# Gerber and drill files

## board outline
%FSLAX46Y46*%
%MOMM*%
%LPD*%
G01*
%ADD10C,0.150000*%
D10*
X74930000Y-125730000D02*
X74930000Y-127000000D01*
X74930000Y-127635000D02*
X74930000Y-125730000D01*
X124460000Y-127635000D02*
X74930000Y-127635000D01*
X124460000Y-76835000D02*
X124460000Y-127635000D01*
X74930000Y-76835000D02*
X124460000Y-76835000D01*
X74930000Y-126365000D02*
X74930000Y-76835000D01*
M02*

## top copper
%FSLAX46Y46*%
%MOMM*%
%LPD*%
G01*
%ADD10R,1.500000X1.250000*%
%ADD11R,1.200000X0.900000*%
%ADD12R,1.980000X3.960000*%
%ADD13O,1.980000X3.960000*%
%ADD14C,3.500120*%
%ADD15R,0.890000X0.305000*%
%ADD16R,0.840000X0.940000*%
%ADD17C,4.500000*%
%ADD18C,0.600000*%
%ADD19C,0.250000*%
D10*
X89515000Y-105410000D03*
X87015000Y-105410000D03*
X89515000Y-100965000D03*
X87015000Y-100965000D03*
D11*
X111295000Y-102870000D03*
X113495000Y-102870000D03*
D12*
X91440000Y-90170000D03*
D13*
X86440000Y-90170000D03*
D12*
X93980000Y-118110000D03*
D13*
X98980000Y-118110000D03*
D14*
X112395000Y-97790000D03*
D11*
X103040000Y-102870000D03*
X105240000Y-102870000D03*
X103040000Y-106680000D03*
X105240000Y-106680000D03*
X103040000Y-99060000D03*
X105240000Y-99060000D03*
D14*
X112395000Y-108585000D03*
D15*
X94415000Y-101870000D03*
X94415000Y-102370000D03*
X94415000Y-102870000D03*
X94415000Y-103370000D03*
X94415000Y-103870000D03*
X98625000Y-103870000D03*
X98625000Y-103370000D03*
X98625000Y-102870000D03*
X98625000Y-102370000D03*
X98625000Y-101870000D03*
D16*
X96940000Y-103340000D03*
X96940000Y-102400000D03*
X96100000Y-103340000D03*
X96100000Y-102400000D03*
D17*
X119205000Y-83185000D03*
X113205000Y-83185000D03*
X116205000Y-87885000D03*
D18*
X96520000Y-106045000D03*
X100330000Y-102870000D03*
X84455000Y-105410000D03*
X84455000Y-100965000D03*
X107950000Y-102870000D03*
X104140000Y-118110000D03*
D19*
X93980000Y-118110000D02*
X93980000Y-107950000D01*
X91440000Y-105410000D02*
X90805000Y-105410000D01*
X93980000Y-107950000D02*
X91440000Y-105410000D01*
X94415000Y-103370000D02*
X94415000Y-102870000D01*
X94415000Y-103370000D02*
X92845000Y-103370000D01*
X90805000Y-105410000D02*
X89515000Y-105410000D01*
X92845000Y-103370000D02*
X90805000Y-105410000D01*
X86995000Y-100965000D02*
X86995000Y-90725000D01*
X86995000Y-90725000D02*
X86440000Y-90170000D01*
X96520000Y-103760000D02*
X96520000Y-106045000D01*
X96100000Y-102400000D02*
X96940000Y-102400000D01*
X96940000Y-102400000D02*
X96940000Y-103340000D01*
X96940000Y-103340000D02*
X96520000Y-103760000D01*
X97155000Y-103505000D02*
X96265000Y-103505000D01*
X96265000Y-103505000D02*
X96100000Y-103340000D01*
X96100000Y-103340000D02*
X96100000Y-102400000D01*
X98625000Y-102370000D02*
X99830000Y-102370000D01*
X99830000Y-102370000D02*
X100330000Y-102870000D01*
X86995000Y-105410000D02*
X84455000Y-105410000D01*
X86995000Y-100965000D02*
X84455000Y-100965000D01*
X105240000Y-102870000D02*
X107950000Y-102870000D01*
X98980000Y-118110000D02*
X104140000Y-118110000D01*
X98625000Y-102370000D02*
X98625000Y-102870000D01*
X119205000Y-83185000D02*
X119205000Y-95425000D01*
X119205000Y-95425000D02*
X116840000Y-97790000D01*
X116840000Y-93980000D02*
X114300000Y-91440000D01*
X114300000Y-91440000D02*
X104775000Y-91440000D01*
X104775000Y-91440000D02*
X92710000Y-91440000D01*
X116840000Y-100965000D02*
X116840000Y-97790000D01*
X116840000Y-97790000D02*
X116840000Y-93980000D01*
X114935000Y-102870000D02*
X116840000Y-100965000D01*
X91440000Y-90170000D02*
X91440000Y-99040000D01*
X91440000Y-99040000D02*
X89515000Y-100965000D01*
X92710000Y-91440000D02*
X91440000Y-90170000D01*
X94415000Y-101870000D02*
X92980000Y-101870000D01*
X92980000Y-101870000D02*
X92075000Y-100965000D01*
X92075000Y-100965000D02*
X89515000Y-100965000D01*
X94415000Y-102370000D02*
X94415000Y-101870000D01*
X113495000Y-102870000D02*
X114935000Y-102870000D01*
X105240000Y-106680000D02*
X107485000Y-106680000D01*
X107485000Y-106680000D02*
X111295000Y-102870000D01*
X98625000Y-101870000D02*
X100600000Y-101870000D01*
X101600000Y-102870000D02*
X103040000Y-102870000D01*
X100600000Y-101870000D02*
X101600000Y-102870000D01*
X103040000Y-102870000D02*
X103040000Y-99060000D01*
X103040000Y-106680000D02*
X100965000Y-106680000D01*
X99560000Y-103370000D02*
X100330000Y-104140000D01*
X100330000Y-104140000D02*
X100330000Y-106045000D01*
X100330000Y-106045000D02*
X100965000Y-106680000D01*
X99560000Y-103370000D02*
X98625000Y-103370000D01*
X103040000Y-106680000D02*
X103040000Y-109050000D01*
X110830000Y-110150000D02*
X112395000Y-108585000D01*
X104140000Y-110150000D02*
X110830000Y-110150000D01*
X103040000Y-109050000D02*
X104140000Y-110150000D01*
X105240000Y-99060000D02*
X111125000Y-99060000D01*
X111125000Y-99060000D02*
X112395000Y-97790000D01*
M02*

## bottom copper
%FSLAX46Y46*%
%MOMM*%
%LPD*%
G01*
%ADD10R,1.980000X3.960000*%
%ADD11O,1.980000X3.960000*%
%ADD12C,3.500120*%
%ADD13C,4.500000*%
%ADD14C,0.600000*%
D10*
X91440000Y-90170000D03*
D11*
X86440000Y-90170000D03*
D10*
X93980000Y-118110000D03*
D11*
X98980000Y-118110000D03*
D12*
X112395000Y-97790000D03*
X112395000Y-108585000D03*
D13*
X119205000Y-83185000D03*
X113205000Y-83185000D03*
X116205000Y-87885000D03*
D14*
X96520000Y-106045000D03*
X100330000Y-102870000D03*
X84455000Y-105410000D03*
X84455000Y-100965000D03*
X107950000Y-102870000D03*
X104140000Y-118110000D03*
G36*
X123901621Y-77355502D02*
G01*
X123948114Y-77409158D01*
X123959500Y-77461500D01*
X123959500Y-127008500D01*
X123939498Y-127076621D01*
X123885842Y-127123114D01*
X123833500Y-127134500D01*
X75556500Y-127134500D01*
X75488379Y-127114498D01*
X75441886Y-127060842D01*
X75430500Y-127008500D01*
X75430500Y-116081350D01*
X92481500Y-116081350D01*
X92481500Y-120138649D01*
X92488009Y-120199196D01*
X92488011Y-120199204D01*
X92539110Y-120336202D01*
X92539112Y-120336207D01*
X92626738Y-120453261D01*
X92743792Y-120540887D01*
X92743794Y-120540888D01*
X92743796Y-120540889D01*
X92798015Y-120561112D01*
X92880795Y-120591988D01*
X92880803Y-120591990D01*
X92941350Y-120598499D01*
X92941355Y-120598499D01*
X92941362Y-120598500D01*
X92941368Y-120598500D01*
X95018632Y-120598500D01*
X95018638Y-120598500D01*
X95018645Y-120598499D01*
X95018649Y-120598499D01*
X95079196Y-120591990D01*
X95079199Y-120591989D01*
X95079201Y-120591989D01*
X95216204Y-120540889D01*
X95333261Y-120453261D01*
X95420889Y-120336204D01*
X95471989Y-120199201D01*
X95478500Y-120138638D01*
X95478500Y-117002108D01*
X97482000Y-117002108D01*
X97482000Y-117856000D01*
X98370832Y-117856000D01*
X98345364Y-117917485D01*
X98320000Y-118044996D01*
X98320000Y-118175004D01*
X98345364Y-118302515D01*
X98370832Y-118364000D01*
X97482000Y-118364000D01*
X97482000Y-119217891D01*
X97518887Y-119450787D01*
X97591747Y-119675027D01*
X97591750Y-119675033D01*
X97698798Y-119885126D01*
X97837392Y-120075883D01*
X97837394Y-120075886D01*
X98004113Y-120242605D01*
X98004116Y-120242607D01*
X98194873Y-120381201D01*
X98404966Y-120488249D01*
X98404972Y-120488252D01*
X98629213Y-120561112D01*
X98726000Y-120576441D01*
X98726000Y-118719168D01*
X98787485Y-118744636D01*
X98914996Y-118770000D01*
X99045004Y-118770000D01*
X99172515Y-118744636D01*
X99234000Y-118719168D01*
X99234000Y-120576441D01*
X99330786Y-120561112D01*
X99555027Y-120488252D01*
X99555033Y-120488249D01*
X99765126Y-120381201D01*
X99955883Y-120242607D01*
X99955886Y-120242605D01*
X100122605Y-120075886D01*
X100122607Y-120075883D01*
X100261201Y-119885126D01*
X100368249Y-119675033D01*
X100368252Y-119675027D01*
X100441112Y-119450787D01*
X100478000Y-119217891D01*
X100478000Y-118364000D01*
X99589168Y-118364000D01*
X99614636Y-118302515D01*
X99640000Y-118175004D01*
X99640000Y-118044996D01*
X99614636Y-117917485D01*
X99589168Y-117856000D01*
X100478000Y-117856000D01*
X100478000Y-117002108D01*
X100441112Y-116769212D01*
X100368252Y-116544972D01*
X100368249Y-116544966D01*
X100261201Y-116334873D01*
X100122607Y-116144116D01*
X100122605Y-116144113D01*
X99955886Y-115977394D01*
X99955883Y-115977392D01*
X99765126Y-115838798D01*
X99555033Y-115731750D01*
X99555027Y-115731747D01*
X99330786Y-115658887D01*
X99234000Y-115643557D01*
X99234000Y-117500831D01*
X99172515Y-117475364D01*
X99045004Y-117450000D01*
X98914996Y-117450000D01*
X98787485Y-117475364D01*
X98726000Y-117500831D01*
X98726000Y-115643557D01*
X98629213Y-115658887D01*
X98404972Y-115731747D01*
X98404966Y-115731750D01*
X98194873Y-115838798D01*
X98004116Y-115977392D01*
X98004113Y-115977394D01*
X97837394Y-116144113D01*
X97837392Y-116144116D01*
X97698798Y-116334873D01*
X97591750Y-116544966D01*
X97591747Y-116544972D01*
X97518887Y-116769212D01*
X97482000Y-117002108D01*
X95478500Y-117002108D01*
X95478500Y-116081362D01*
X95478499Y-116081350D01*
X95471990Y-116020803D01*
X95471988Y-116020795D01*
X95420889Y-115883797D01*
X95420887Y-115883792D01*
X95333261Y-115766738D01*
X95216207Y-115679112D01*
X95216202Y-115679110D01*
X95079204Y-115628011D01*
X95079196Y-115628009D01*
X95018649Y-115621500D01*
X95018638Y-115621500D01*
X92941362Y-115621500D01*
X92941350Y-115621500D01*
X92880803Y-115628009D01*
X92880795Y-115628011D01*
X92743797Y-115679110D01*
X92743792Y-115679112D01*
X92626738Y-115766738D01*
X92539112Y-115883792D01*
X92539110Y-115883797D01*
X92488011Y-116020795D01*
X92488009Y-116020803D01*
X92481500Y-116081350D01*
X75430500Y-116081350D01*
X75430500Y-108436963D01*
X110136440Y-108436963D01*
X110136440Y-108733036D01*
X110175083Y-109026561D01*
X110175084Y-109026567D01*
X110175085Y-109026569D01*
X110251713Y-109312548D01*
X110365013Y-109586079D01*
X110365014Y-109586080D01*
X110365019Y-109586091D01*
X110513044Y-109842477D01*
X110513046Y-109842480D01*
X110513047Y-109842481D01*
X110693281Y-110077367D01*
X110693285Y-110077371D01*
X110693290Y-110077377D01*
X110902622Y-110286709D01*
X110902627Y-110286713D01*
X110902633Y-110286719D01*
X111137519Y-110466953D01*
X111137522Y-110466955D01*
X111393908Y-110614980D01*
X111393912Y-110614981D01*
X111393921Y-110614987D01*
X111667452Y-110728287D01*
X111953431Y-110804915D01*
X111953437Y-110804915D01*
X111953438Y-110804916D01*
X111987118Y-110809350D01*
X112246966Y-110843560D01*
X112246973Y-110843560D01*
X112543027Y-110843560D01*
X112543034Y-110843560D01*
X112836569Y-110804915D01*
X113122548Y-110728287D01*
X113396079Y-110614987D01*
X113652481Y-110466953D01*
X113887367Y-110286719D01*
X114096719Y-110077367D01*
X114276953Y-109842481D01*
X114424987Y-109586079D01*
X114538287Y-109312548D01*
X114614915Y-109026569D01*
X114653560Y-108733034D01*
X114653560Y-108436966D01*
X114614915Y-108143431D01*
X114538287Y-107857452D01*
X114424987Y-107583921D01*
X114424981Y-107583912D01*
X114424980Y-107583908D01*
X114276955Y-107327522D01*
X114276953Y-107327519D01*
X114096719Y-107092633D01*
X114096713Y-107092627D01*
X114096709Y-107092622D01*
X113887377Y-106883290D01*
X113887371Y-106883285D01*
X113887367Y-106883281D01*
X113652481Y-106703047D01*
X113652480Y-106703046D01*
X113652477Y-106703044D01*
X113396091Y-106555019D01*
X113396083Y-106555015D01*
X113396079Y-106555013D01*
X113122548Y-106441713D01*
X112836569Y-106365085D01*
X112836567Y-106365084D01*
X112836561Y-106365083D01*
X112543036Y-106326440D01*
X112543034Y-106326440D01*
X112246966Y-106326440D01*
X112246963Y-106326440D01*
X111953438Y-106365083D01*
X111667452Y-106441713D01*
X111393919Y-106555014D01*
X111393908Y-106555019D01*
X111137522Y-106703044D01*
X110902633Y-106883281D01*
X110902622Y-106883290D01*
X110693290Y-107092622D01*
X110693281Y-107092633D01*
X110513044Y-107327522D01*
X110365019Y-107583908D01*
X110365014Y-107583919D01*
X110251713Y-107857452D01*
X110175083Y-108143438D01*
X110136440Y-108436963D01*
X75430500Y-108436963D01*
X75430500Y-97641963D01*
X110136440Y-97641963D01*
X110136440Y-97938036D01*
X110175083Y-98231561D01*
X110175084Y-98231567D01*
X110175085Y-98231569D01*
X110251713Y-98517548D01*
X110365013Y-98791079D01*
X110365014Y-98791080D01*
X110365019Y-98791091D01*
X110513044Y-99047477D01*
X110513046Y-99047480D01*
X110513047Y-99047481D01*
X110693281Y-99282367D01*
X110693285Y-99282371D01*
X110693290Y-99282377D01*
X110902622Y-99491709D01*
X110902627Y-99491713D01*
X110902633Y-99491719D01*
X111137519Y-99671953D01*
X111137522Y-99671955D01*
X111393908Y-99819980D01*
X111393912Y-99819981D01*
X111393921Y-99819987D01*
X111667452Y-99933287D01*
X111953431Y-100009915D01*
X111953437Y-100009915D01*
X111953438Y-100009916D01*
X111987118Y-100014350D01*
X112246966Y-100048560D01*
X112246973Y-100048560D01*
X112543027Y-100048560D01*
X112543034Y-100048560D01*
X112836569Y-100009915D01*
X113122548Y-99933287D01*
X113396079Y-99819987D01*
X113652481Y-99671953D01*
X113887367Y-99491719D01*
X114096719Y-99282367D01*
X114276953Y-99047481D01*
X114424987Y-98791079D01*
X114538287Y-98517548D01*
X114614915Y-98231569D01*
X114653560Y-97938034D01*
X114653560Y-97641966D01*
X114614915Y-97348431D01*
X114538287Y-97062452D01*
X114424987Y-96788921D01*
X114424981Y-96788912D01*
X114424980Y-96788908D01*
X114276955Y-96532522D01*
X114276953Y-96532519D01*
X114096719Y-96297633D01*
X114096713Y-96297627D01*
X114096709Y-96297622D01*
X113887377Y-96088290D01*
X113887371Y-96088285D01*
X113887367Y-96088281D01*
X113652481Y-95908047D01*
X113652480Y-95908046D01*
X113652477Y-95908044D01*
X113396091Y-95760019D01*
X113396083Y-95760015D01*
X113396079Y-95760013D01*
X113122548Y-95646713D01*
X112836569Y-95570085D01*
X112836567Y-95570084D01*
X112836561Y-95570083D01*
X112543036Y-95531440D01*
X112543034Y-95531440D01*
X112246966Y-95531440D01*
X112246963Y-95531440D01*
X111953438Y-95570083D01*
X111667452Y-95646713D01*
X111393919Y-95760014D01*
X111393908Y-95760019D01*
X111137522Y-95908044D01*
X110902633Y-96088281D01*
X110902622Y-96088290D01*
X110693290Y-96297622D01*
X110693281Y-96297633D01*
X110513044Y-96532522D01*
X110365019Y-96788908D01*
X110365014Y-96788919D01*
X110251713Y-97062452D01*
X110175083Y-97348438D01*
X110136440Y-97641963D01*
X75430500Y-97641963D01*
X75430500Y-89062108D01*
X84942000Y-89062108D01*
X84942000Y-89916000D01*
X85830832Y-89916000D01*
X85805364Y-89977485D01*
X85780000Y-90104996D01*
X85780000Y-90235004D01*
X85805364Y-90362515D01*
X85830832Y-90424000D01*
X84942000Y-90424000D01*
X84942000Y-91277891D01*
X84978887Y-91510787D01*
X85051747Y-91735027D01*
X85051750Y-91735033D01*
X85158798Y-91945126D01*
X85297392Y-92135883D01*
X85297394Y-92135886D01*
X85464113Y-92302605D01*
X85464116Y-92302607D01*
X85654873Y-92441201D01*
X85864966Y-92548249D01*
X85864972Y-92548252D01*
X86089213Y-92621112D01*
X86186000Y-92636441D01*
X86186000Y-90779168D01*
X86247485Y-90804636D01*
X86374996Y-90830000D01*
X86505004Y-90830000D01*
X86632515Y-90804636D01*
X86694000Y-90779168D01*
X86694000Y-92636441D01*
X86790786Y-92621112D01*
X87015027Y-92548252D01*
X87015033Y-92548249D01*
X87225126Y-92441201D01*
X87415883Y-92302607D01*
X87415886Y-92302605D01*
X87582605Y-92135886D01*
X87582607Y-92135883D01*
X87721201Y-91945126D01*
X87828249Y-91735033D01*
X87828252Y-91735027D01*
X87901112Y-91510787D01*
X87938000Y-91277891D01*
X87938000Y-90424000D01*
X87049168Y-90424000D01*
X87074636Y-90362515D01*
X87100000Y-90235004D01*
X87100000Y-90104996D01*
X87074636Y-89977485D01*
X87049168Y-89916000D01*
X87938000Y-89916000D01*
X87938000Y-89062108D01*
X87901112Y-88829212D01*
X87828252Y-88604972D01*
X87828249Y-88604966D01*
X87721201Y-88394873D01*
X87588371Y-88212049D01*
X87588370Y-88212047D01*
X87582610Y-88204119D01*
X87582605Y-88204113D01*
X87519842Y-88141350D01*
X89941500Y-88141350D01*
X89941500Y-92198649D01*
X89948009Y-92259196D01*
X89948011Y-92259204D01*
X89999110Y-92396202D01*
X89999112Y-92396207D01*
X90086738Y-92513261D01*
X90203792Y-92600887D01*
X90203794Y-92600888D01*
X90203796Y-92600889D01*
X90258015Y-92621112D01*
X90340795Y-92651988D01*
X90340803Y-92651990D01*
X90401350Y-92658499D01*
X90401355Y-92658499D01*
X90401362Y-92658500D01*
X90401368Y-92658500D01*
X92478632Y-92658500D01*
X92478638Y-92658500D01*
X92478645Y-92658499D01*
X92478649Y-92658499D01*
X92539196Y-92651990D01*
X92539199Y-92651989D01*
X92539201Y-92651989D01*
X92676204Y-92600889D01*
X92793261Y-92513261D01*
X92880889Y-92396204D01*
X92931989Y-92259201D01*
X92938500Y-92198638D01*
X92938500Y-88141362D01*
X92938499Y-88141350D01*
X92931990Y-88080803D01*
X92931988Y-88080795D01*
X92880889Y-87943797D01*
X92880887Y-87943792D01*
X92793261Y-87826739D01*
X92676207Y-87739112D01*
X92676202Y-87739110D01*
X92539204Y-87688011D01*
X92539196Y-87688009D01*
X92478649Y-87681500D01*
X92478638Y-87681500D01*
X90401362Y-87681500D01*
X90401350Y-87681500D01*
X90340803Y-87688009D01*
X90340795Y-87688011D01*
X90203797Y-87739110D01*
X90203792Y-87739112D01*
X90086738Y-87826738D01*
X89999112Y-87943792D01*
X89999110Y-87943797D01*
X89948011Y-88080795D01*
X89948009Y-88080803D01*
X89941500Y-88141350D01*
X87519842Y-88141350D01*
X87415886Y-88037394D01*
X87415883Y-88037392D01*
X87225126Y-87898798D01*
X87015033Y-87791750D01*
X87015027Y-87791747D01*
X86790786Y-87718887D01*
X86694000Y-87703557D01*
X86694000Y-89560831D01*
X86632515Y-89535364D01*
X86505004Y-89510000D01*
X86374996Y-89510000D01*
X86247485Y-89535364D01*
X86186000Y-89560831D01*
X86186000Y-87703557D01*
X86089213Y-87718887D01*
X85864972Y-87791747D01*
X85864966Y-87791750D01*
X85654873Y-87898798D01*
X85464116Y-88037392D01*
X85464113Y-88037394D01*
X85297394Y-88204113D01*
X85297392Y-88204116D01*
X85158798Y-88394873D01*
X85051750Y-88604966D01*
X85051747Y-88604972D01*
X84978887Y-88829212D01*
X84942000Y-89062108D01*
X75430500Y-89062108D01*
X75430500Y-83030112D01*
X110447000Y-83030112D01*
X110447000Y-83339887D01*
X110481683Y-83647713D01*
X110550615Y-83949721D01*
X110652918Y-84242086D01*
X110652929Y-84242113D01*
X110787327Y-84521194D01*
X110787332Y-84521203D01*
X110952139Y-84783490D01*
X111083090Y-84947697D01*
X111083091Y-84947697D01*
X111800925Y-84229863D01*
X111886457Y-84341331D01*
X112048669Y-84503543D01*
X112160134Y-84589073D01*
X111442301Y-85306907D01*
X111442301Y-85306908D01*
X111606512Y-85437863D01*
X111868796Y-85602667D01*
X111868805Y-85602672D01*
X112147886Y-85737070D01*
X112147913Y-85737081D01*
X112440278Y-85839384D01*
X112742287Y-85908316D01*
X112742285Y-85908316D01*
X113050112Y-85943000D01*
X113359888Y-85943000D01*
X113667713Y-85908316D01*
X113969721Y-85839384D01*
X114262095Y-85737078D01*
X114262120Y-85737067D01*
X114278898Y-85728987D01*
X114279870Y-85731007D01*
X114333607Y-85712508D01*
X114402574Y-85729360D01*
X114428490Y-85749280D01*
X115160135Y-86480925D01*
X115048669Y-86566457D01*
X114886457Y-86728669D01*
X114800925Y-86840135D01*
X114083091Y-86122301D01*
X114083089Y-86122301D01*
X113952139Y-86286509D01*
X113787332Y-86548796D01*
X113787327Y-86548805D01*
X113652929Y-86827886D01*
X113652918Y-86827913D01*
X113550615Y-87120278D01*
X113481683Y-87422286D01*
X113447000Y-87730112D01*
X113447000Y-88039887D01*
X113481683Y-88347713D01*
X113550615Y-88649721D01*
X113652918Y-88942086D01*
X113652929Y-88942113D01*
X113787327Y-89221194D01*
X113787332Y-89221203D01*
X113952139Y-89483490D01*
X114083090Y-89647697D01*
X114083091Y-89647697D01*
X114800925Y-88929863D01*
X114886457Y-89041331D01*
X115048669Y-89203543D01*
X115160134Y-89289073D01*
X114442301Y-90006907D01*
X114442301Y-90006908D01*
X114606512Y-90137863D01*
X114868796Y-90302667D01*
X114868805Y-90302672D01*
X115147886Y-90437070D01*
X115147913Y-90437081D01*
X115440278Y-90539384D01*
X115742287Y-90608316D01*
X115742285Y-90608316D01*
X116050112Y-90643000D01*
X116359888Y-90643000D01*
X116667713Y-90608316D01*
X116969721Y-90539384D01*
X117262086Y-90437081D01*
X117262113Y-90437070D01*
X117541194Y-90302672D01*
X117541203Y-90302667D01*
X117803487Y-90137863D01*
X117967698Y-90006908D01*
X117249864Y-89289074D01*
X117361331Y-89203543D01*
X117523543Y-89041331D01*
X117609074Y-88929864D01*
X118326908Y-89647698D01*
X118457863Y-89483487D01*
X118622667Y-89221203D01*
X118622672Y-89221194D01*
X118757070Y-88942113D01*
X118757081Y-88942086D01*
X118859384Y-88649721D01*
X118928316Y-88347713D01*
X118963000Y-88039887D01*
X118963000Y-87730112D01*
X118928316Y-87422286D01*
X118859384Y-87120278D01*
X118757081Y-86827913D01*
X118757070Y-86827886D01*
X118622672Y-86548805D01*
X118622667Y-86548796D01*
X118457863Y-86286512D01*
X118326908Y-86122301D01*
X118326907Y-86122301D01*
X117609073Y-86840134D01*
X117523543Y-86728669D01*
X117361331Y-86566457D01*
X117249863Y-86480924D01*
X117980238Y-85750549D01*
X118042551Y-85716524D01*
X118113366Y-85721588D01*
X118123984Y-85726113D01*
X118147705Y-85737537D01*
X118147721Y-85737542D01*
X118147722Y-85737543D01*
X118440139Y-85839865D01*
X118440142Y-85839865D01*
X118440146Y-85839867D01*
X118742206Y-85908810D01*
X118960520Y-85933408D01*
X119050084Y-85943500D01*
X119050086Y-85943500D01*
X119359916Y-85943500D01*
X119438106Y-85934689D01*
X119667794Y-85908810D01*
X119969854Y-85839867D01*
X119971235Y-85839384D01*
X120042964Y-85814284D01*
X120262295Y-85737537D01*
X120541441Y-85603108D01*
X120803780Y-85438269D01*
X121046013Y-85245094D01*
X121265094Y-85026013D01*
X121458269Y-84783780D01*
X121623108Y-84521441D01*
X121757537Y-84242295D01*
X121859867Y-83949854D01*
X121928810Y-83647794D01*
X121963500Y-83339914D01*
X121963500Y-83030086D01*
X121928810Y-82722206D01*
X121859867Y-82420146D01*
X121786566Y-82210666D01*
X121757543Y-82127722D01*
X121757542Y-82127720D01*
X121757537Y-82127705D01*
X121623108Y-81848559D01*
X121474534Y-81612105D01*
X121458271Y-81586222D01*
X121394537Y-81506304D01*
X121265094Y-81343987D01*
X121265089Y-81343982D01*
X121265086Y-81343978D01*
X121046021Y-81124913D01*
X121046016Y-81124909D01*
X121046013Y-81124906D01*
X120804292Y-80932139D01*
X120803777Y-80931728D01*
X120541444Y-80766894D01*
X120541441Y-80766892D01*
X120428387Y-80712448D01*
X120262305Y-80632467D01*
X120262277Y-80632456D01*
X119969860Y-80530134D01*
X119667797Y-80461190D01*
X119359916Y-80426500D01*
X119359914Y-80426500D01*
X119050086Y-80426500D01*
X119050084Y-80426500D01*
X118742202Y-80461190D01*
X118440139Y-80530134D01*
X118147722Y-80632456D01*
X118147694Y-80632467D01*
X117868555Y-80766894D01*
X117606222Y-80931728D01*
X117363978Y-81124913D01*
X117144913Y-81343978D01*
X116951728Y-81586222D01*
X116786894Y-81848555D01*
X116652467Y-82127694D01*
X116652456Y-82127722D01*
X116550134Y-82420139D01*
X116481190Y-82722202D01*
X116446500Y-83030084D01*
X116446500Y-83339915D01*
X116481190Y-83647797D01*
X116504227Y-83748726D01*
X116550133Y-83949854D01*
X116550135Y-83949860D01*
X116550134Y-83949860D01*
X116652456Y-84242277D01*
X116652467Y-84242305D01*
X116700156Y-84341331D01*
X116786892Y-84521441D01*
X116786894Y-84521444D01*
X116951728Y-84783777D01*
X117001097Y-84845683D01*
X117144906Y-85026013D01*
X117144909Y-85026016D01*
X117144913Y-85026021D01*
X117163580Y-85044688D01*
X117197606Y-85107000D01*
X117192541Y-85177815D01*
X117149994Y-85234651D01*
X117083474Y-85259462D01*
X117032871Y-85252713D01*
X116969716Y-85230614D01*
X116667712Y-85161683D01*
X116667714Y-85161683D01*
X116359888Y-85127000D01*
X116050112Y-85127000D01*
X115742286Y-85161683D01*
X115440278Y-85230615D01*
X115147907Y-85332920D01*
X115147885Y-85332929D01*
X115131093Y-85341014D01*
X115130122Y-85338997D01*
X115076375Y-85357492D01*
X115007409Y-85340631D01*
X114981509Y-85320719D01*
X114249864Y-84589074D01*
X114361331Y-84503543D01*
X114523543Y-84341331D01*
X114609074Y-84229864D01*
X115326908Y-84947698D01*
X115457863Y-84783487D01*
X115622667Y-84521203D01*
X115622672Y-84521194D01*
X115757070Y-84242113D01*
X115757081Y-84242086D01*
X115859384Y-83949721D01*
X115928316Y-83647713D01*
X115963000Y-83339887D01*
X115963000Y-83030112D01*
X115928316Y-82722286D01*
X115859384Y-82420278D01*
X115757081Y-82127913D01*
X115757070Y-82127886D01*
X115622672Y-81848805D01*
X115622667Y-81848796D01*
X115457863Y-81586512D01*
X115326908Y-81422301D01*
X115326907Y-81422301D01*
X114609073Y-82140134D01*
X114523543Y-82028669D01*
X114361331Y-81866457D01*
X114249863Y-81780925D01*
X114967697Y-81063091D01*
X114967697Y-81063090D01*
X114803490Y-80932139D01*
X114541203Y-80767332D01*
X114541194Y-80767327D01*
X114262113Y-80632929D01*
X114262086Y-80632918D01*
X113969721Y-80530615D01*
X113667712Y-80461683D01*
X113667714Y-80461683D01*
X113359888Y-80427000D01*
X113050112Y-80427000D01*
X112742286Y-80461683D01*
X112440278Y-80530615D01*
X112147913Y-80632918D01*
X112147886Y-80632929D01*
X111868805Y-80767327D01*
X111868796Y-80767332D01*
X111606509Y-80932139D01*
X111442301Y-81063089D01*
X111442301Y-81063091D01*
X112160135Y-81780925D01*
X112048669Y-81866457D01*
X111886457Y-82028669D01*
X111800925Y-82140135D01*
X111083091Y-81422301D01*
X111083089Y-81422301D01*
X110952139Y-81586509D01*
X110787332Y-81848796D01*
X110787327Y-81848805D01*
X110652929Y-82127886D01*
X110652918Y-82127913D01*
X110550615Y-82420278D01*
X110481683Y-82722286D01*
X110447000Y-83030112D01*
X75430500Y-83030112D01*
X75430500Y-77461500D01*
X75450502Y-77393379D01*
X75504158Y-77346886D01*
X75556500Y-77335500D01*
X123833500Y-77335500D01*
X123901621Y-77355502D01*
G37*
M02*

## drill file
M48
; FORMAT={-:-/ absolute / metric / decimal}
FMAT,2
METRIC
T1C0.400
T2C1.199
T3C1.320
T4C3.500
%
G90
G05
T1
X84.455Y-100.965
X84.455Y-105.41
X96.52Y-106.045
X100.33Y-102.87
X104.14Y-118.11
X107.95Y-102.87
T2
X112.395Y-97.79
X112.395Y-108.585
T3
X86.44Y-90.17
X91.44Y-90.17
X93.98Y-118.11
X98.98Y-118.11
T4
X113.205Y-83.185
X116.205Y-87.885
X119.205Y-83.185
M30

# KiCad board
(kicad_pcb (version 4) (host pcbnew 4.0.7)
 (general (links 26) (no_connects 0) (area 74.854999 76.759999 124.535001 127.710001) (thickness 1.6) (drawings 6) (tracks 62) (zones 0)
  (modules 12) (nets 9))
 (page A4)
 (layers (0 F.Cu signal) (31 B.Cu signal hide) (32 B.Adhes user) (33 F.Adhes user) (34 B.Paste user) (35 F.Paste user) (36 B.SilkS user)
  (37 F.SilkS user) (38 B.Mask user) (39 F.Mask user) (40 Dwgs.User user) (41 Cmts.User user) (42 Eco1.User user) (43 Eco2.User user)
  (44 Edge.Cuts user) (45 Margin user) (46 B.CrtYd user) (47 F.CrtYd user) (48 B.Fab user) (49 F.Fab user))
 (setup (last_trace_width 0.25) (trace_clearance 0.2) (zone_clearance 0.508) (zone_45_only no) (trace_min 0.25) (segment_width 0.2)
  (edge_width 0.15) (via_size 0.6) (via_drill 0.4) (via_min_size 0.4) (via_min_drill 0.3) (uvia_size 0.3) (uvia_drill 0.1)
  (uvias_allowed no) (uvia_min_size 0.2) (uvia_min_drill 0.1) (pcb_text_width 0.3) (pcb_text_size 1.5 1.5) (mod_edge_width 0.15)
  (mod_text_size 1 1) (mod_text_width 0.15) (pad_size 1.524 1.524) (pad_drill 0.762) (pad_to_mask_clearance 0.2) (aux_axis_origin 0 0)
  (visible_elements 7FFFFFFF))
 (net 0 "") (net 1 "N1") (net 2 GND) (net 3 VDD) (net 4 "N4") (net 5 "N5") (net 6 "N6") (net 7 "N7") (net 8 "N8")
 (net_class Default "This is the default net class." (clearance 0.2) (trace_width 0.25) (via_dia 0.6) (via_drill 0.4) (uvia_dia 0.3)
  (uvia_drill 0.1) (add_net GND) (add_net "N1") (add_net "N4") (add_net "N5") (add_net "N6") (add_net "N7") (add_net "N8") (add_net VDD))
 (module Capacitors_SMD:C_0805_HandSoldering (layer F.Cu) (at 88.265 105.41 180)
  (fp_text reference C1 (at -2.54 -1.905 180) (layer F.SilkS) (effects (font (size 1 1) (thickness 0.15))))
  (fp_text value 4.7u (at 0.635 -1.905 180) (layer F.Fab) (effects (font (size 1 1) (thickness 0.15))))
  (pad 1 smd rect (at -1.25 0 180) (size 1.5 1.25) (layers F.Cu F.Paste F.Mask) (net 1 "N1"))
  (pad 2 smd rect (at 1.25 0 180) (size 1.5 1.25) (layers F.Cu F.Paste F.Mask) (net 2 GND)))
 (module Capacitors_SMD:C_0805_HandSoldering (layer F.Cu) (at 88.265 100.965 180)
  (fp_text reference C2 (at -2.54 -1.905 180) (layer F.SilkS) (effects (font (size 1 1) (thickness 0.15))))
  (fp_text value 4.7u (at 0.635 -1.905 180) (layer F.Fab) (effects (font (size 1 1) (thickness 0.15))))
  (pad 1 smd rect (at -1.25 0 180) (size 1.5 1.25) (layers F.Cu F.Paste F.Mask) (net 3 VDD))
  (pad 2 smd rect (at 1.25 0 180) (size 1.5 1.25) (layers F.Cu F.Paste F.Mask) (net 2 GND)))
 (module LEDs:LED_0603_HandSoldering (layer F.Cu) (at 112.395 102.87)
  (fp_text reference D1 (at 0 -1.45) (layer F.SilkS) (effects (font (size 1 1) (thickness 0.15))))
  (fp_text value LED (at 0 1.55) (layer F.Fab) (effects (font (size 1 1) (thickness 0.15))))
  (pad 1 smd rect (at -1.1 0) (size 1.2 0.9) (layers F.Cu F.Paste F.Mask) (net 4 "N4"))
  (pad 2 smd rect (at 1.1 0) (size 1.2 0.9) (layers F.Cu F.Paste F.Mask) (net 3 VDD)))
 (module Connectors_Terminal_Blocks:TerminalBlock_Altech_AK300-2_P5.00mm (layer F.Cu) (at 91.44 90.17 180)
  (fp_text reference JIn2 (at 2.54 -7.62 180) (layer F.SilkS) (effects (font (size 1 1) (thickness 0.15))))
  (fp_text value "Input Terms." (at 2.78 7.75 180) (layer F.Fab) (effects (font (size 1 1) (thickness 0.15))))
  (pad 1 thru_hole rect (at 0 0 180) (size 1.98 3.96) (drill 1.32) (layers *.Cu *.Mask) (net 3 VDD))
  (pad 2 thru_hole oval (at 5 0 180) (size 1.98 3.96) (drill 1.32) (layers *.Cu *.Mask) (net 2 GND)))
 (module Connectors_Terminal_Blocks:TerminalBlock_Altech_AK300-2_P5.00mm (layer F.Cu) (at 93.98 118.11)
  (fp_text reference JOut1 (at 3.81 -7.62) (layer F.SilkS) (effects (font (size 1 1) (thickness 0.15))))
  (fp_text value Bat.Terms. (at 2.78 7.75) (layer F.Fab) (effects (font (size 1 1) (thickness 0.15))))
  (pad 1 thru_hole rect (at 0 0) (size 1.98 3.96) (drill 1.32) (layers *.Cu *.Mask) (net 1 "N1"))
  (pad 2 thru_hole oval (at 5 0) (size 1.98 3.96) (drill 1.32) (layers *.Cu *.Mask) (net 2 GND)))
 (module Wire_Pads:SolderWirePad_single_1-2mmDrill (layer F.Cu) (at 112.395 97.79)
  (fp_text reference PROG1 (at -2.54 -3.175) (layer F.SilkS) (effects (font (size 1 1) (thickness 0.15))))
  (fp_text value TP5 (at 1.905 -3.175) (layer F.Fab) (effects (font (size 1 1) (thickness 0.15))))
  (pad 1 thru_hole circle (at 0 0) (size 3.50012 3.50012) (drill 1.19888) (layers *.Cu *.Mask) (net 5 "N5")))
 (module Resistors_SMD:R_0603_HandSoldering (layer F.Cu) (at 104.14 102.87)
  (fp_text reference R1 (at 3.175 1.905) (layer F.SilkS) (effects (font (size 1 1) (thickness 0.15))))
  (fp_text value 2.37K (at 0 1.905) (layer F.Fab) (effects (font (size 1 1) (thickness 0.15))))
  (pad 1 smd rect (at -1.1 0) (size 1.2 0.9) (layers F.Cu F.Paste F.Mask) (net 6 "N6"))
  (pad 2 smd rect (at 1.1 0) (size 1.2 0.9) (layers F.Cu F.Paste F.Mask) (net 2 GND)))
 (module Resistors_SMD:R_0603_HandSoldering (layer F.Cu) (at 104.14 106.68)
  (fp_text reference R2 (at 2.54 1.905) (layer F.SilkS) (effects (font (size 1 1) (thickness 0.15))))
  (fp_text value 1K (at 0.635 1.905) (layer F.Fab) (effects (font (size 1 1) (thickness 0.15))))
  (pad 1 smd rect (at -1.1 0) (size 1.2 0.9) (layers F.Cu F.Paste F.Mask) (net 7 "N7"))
  (pad 2 smd rect (at 1.1 0) (size 1.2 0.9) (layers F.Cu F.Paste F.Mask) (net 4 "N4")))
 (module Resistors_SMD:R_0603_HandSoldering (layer F.Cu) (at 104.14 99.06)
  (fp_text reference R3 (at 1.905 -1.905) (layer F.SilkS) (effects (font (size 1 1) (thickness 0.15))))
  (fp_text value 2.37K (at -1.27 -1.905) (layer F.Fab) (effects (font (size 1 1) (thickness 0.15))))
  (pad 1 smd rect (at -1.1 0) (size 1.2 0.9) (layers F.Cu F.Paste F.Mask) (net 6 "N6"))
  (pad 2 smd rect (at 1.1 0) (size 1.2 0.9) (layers F.Cu F.Paste F.Mask) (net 5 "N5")))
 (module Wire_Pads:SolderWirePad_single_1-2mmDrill (layer F.Cu) (at 112.395 108.585)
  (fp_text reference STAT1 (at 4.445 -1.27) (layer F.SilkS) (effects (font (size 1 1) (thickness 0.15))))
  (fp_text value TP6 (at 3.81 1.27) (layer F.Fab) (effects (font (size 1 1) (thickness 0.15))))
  (pad 1 thru_hole circle (at 0 0) (size 3.50012 3.50012) (drill 1.19888) (layers *.Cu *.Mask) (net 7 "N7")))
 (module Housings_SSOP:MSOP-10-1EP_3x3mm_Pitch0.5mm (layer F.Cu) (at 96.52 102.87)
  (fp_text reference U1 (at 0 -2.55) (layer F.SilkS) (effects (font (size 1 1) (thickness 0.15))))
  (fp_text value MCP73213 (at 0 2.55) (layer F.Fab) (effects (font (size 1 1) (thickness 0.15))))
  (pad 1 smd rect (at -2.105 -1) (size 0.89 0.305) (layers F.Cu F.Paste F.Mask) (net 3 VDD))
  (pad 2 smd rect (at -2.105 -0.5) (size 0.89 0.305) (layers F.Cu F.Paste F.Mask) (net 3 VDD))
  (pad 3 smd rect (at -2.105 0) (size 0.89 0.305) (layers F.Cu F.Paste F.Mask) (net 1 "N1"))
  (pad 4 smd rect (at -2.105 0.5) (size 0.89 0.305) (layers F.Cu F.Paste F.Mask) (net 1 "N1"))
  (pad 5 smd rect (at -2.105 1) (size 0.89 0.305) (layers F.Cu F.Paste F.Mask) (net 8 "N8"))
  (pad 6 smd rect (at 2.105 1) (size 0.89 0.305) (layers F.Cu F.Paste F.Mask))
  (pad 7 smd rect (at 2.105 0.5) (size 0.89 0.305) (layers F.Cu F.Paste F.Mask) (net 7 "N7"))
  (pad 8 smd rect (at 2.105 0) (size 0.89 0.305) (layers F.Cu F.Paste F.Mask) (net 2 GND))
  (pad 9 smd rect (at 2.105 -0.5) (size 0.89 0.305) (layers F.Cu F.Paste F.Mask) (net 2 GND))
  (pad 10 smd rect (at 2.105 -1) (size 0.89 0.305) (layers F.Cu F.Paste F.Mask) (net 6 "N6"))
  (pad 11 smd rect (at 0.42 0.47) (size 0.84 0.94) (layers F.Cu F.Paste F.Mask) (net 2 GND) (solder_paste_margin_ratio -0.2))
  (pad 11 smd rect (at 0.42 -0.47) (size 0.84 0.94) (layers F.Cu F.Paste F.Mask) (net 2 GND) (solder_paste_margin_ratio -0.2))
  (pad 11 smd rect (at -0.42 0.47) (size 0.84 0.94) (layers F.Cu F.Paste F.Mask) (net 2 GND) (solder_paste_margin_ratio -0.2))
  (pad 11 smd rect (at -0.42 -0.47) (size 0.84 0.94) (layers F.Cu F.Paste F.Mask) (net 2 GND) (solder_paste_margin_ratio -0.2)))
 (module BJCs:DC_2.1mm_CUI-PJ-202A (layer F.Cu) (at 116.205 83.185 180)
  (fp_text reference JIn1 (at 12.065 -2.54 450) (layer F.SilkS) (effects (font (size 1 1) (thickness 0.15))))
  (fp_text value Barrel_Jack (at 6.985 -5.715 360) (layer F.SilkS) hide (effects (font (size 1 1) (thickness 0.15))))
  (pad 1 thru_hole circle (at -3 0 180) (size 4.5 4.5) (drill 3.5) (layers *.Cu *.Mask F.SilkS) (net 3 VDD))
  (pad 2 thru_hole circle (at 3 0 180) (size 4.5 4.5) (drill 3.5) (layers *.Cu *.Mask F.SilkS) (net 2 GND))
  (pad 3 thru_hole circle (at 0 -4.7 180) (size 4.5 4.5) (drill 3.5) (layers *.Cu *.Mask F.SilkS) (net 2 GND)))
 (gr_line (start 74.93 125.73) (end 74.93 127) (angle 90) (layer Edge.Cuts) (width 0.15))
 (gr_line (start 74.93 127.635) (end 74.93 125.73) (angle 90) (layer Edge.Cuts) (width 0.15))
 (gr_line (start 124.46 127.635) (end 74.93 127.635) (angle 90) (layer Edge.Cuts) (width 0.15))
 (gr_line (start 124.46 76.835) (end 124.46 127.635) (angle 90) (layer Edge.Cuts) (width 0.15))
 (gr_line (start 74.93 76.835) (end 124.46 76.835) (angle 90) (layer Edge.Cuts) (width 0.15))
 (gr_line (start 74.93 126.365) (end 74.93 76.835) (angle 90) (layer Edge.Cuts) (width 0.15))
 (segment (start 93.98 118.11) (end 93.98 107.95) (width 0.25) (layer F.Cu) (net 1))
 (segment (start 91.44 105.41) (end 90.805 105.41) (width 0.25) (layer F.Cu) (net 1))
 (segment (start 93.98 107.95) (end 91.44 105.41) (width 0.25) (layer F.Cu) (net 1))
 (segment (start 94.415 103.37) (end 94.415 102.87) (width 0.25) (layer F.Cu) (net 1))
 (segment (start 94.415 103.37) (end 92.845 103.37) (width 0.25) (layer F.Cu) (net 1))
 (segment (start 90.805 105.41) (end 89.515 105.41) (width 0.25) (layer F.Cu) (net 1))
 (segment (start 92.845 103.37) (end 90.805 105.41) (width 0.25) (layer F.Cu) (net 1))
 (segment (start 86.995 100.965) (end 86.995 90.725) (width 0.25) (layer F.Cu) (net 2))
 (segment (start 86.995 90.725) (end 86.44 90.17) (width 0.25) (layer F.Cu) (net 2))
 (segment (start 96.52 103.76) (end 96.52 106.045) (width 0.25) (layer F.Cu) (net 2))
 (via (at 96.52 106.045) (size 0.6) (drill 0.4) (layers F.Cu B.Cu) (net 2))
 (segment (start 96.1 102.4) (end 96.94 102.4) (width 0.25) (layer F.Cu) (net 2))
 (segment (start 96.94 102.4) (end 96.94 103.34) (width 0.25) (layer F.Cu) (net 2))
 (segment (start 96.94 103.34) (end 96.52 103.76) (width 0.25) (layer F.Cu) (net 2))
 (segment (start 97.155 103.505) (end 96.265 103.505) (width 0.25) (layer F.Cu) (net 2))
 (segment (start 96.265 103.505) (end 96.1 103.34) (width 0.25) (layer F.Cu) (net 2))
 (segment (start 96.1 103.34) (end 96.1 102.4) (width 0.25) (layer F.Cu) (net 2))
 (segment (start 98.625 102.37) (end 99.83 102.37) (width 0.25) (layer F.Cu) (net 2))
 (via (at 100.33 102.87) (size 0.6) (drill 0.4) (layers F.Cu B.Cu) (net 2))
 (segment (start 99.83 102.37) (end 100.33 102.87) (width 0.25) (layer F.Cu) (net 2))
 (segment (start 86.995 105.41) (end 84.455 105.41) (width 0.25) (layer F.Cu) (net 2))
 (via (at 84.455 105.41) (size 0.6) (drill 0.4) (layers F.Cu B.Cu) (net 2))
 (segment (start 86.995 100.965) (end 84.455 100.965) (width 0.25) (layer F.Cu) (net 2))
 (via (at 84.455 100.965) (size 0.6) (drill 0.4) (layers F.Cu B.Cu) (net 2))
 (segment (start 105.24 102.87) (end 107.95 102.87) (width 0.25) (layer F.Cu) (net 2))
 (via (at 107.95 102.87) (size 0.6) (drill 0.4) (layers F.Cu B.Cu) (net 2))
 (segment (start 98.98 118.11) (end 104.14 118.11) (width 0.25) (layer F.Cu) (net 2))
 (via (at 104.14 118.11) (size 0.6) (drill 0.4) (layers F.Cu B.Cu) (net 2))
 (segment (start 98.625 102.37) (end 98.625 102.87) (width 0.25) (layer F.Cu) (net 2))
 (segment (start 119.205 83.185) (end 119.205 95.425) (width 0.25) (layer F.Cu) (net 3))
 (segment (start 119.205 95.425) (end 116.84 97.79) (width 0.25) (layer F.Cu) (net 3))
 (segment (start 116.84 93.98) (end 114.3 91.44) (width 0.25) (layer F.Cu) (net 3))
 (segment (start 114.3 91.44) (end 104.775 91.44) (width 0.25) (layer F.Cu) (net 3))
 (segment (start 104.775 91.44) (end 92.71 91.44) (width 0.25) (layer F.Cu) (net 3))
 (segment (start 116.84 100.965) (end 116.84 97.79) (width 0.25) (layer F.Cu) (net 3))
 (segment (start 116.84 97.79) (end 116.84 93.98) (width 0.25) (layer F.Cu) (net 3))
 (segment (start 114.935 102.87) (end 116.84 100.965) (width 0.25) (layer F.Cu) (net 3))
 (segment (start 91.44 90.17) (end 91.44 99.04) (width 0.25) (layer F.Cu) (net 3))
 (segment (start 91.44 99.04) (end 89.515 100.965) (width 0.25) (layer F.Cu) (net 3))
 (segment (start 92.71 91.44) (end 91.44 90.17) (width 0.25) (layer F.Cu) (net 3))
 (segment (start 94.415 101.87) (end 92.98 101.87) (width 0.25) (layer F.Cu) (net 3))
 (segment (start 92.98 101.87) (end 92.075 100.965) (width 0.25) (layer F.Cu) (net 3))
 (segment (start 92.075 100.965) (end 89.515 100.965) (width 0.25) (layer F.Cu) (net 3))
 (segment (start 94.415 102.37) (end 94.415 101.87) (width 0.25) (layer F.Cu) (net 3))
 (segment (start 113.495 102.87) (end 114.935 102.87) (width 0.25) (layer F.Cu) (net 3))
 (segment (start 105.24 106.68) (end 107.485 106.68) (width 0.25) (layer F.Cu) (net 4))
 (segment (start 107.485 106.68) (end 111.295 102.87) (width 0.25) (layer F.Cu) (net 4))
 (segment (start 98.625 101.87) (end 100.6 101.87) (width 0.25) (layer F.Cu) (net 6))
 (segment (start 101.6 102.87) (end 103.04 102.87) (width 0.25) (layer F.Cu) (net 6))
 (segment (start 100.6 101.87) (end 101.6 102.87) (width 0.25) (layer F.Cu) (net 6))
 (segment (start 103.04 102.87) (end 103.04 99.06) (width 0.25) (layer F.Cu) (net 6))
 (segment (start 103.04 106.68) (end 100.965 106.68) (width 0.25) (layer F.Cu) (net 7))
 (segment (start 99.56 103.37) (end 100.33 104.14) (width 0.25) (layer F.Cu) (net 7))
 (segment (start 100.33 104.14) (end 100.33 106.045) (width 0.25) (layer F.Cu) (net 7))
 (segment (start 100.33 106.045) (end 100.965 106.68) (width 0.25) (layer F.Cu) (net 7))
 (segment (start 99.56 103.37) (end 98.625 103.37) (width 0.25) (layer F.Cu) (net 7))
 (segment (start 103.04 106.68) (end 103.04 109.05) (width 0.25) (layer F.Cu) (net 7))
 (segment (start 110.83 110.15) (end 112.395 108.585) (width 0.25) (layer F.Cu) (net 7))
 (segment (start 104.14 110.15) (end 110.83 110.15) (width 0.25) (layer F.Cu) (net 7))
 (segment (start 103.04 109.05) (end 104.14 110.15) (width 0.25) (layer F.Cu) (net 7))
 (segment (start 105.24 99.06) (end 111.125 99.06) (width 0.25) (layer F.Cu) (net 5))
 (segment (start 111.125 99.06) (end 112.395 97.79) (width 0.25) (layer F.Cu) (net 5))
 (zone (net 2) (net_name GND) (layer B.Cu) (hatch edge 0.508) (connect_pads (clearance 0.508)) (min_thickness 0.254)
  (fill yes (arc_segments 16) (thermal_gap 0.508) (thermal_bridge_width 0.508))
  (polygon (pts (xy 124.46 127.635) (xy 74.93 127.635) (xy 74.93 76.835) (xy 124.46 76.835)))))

